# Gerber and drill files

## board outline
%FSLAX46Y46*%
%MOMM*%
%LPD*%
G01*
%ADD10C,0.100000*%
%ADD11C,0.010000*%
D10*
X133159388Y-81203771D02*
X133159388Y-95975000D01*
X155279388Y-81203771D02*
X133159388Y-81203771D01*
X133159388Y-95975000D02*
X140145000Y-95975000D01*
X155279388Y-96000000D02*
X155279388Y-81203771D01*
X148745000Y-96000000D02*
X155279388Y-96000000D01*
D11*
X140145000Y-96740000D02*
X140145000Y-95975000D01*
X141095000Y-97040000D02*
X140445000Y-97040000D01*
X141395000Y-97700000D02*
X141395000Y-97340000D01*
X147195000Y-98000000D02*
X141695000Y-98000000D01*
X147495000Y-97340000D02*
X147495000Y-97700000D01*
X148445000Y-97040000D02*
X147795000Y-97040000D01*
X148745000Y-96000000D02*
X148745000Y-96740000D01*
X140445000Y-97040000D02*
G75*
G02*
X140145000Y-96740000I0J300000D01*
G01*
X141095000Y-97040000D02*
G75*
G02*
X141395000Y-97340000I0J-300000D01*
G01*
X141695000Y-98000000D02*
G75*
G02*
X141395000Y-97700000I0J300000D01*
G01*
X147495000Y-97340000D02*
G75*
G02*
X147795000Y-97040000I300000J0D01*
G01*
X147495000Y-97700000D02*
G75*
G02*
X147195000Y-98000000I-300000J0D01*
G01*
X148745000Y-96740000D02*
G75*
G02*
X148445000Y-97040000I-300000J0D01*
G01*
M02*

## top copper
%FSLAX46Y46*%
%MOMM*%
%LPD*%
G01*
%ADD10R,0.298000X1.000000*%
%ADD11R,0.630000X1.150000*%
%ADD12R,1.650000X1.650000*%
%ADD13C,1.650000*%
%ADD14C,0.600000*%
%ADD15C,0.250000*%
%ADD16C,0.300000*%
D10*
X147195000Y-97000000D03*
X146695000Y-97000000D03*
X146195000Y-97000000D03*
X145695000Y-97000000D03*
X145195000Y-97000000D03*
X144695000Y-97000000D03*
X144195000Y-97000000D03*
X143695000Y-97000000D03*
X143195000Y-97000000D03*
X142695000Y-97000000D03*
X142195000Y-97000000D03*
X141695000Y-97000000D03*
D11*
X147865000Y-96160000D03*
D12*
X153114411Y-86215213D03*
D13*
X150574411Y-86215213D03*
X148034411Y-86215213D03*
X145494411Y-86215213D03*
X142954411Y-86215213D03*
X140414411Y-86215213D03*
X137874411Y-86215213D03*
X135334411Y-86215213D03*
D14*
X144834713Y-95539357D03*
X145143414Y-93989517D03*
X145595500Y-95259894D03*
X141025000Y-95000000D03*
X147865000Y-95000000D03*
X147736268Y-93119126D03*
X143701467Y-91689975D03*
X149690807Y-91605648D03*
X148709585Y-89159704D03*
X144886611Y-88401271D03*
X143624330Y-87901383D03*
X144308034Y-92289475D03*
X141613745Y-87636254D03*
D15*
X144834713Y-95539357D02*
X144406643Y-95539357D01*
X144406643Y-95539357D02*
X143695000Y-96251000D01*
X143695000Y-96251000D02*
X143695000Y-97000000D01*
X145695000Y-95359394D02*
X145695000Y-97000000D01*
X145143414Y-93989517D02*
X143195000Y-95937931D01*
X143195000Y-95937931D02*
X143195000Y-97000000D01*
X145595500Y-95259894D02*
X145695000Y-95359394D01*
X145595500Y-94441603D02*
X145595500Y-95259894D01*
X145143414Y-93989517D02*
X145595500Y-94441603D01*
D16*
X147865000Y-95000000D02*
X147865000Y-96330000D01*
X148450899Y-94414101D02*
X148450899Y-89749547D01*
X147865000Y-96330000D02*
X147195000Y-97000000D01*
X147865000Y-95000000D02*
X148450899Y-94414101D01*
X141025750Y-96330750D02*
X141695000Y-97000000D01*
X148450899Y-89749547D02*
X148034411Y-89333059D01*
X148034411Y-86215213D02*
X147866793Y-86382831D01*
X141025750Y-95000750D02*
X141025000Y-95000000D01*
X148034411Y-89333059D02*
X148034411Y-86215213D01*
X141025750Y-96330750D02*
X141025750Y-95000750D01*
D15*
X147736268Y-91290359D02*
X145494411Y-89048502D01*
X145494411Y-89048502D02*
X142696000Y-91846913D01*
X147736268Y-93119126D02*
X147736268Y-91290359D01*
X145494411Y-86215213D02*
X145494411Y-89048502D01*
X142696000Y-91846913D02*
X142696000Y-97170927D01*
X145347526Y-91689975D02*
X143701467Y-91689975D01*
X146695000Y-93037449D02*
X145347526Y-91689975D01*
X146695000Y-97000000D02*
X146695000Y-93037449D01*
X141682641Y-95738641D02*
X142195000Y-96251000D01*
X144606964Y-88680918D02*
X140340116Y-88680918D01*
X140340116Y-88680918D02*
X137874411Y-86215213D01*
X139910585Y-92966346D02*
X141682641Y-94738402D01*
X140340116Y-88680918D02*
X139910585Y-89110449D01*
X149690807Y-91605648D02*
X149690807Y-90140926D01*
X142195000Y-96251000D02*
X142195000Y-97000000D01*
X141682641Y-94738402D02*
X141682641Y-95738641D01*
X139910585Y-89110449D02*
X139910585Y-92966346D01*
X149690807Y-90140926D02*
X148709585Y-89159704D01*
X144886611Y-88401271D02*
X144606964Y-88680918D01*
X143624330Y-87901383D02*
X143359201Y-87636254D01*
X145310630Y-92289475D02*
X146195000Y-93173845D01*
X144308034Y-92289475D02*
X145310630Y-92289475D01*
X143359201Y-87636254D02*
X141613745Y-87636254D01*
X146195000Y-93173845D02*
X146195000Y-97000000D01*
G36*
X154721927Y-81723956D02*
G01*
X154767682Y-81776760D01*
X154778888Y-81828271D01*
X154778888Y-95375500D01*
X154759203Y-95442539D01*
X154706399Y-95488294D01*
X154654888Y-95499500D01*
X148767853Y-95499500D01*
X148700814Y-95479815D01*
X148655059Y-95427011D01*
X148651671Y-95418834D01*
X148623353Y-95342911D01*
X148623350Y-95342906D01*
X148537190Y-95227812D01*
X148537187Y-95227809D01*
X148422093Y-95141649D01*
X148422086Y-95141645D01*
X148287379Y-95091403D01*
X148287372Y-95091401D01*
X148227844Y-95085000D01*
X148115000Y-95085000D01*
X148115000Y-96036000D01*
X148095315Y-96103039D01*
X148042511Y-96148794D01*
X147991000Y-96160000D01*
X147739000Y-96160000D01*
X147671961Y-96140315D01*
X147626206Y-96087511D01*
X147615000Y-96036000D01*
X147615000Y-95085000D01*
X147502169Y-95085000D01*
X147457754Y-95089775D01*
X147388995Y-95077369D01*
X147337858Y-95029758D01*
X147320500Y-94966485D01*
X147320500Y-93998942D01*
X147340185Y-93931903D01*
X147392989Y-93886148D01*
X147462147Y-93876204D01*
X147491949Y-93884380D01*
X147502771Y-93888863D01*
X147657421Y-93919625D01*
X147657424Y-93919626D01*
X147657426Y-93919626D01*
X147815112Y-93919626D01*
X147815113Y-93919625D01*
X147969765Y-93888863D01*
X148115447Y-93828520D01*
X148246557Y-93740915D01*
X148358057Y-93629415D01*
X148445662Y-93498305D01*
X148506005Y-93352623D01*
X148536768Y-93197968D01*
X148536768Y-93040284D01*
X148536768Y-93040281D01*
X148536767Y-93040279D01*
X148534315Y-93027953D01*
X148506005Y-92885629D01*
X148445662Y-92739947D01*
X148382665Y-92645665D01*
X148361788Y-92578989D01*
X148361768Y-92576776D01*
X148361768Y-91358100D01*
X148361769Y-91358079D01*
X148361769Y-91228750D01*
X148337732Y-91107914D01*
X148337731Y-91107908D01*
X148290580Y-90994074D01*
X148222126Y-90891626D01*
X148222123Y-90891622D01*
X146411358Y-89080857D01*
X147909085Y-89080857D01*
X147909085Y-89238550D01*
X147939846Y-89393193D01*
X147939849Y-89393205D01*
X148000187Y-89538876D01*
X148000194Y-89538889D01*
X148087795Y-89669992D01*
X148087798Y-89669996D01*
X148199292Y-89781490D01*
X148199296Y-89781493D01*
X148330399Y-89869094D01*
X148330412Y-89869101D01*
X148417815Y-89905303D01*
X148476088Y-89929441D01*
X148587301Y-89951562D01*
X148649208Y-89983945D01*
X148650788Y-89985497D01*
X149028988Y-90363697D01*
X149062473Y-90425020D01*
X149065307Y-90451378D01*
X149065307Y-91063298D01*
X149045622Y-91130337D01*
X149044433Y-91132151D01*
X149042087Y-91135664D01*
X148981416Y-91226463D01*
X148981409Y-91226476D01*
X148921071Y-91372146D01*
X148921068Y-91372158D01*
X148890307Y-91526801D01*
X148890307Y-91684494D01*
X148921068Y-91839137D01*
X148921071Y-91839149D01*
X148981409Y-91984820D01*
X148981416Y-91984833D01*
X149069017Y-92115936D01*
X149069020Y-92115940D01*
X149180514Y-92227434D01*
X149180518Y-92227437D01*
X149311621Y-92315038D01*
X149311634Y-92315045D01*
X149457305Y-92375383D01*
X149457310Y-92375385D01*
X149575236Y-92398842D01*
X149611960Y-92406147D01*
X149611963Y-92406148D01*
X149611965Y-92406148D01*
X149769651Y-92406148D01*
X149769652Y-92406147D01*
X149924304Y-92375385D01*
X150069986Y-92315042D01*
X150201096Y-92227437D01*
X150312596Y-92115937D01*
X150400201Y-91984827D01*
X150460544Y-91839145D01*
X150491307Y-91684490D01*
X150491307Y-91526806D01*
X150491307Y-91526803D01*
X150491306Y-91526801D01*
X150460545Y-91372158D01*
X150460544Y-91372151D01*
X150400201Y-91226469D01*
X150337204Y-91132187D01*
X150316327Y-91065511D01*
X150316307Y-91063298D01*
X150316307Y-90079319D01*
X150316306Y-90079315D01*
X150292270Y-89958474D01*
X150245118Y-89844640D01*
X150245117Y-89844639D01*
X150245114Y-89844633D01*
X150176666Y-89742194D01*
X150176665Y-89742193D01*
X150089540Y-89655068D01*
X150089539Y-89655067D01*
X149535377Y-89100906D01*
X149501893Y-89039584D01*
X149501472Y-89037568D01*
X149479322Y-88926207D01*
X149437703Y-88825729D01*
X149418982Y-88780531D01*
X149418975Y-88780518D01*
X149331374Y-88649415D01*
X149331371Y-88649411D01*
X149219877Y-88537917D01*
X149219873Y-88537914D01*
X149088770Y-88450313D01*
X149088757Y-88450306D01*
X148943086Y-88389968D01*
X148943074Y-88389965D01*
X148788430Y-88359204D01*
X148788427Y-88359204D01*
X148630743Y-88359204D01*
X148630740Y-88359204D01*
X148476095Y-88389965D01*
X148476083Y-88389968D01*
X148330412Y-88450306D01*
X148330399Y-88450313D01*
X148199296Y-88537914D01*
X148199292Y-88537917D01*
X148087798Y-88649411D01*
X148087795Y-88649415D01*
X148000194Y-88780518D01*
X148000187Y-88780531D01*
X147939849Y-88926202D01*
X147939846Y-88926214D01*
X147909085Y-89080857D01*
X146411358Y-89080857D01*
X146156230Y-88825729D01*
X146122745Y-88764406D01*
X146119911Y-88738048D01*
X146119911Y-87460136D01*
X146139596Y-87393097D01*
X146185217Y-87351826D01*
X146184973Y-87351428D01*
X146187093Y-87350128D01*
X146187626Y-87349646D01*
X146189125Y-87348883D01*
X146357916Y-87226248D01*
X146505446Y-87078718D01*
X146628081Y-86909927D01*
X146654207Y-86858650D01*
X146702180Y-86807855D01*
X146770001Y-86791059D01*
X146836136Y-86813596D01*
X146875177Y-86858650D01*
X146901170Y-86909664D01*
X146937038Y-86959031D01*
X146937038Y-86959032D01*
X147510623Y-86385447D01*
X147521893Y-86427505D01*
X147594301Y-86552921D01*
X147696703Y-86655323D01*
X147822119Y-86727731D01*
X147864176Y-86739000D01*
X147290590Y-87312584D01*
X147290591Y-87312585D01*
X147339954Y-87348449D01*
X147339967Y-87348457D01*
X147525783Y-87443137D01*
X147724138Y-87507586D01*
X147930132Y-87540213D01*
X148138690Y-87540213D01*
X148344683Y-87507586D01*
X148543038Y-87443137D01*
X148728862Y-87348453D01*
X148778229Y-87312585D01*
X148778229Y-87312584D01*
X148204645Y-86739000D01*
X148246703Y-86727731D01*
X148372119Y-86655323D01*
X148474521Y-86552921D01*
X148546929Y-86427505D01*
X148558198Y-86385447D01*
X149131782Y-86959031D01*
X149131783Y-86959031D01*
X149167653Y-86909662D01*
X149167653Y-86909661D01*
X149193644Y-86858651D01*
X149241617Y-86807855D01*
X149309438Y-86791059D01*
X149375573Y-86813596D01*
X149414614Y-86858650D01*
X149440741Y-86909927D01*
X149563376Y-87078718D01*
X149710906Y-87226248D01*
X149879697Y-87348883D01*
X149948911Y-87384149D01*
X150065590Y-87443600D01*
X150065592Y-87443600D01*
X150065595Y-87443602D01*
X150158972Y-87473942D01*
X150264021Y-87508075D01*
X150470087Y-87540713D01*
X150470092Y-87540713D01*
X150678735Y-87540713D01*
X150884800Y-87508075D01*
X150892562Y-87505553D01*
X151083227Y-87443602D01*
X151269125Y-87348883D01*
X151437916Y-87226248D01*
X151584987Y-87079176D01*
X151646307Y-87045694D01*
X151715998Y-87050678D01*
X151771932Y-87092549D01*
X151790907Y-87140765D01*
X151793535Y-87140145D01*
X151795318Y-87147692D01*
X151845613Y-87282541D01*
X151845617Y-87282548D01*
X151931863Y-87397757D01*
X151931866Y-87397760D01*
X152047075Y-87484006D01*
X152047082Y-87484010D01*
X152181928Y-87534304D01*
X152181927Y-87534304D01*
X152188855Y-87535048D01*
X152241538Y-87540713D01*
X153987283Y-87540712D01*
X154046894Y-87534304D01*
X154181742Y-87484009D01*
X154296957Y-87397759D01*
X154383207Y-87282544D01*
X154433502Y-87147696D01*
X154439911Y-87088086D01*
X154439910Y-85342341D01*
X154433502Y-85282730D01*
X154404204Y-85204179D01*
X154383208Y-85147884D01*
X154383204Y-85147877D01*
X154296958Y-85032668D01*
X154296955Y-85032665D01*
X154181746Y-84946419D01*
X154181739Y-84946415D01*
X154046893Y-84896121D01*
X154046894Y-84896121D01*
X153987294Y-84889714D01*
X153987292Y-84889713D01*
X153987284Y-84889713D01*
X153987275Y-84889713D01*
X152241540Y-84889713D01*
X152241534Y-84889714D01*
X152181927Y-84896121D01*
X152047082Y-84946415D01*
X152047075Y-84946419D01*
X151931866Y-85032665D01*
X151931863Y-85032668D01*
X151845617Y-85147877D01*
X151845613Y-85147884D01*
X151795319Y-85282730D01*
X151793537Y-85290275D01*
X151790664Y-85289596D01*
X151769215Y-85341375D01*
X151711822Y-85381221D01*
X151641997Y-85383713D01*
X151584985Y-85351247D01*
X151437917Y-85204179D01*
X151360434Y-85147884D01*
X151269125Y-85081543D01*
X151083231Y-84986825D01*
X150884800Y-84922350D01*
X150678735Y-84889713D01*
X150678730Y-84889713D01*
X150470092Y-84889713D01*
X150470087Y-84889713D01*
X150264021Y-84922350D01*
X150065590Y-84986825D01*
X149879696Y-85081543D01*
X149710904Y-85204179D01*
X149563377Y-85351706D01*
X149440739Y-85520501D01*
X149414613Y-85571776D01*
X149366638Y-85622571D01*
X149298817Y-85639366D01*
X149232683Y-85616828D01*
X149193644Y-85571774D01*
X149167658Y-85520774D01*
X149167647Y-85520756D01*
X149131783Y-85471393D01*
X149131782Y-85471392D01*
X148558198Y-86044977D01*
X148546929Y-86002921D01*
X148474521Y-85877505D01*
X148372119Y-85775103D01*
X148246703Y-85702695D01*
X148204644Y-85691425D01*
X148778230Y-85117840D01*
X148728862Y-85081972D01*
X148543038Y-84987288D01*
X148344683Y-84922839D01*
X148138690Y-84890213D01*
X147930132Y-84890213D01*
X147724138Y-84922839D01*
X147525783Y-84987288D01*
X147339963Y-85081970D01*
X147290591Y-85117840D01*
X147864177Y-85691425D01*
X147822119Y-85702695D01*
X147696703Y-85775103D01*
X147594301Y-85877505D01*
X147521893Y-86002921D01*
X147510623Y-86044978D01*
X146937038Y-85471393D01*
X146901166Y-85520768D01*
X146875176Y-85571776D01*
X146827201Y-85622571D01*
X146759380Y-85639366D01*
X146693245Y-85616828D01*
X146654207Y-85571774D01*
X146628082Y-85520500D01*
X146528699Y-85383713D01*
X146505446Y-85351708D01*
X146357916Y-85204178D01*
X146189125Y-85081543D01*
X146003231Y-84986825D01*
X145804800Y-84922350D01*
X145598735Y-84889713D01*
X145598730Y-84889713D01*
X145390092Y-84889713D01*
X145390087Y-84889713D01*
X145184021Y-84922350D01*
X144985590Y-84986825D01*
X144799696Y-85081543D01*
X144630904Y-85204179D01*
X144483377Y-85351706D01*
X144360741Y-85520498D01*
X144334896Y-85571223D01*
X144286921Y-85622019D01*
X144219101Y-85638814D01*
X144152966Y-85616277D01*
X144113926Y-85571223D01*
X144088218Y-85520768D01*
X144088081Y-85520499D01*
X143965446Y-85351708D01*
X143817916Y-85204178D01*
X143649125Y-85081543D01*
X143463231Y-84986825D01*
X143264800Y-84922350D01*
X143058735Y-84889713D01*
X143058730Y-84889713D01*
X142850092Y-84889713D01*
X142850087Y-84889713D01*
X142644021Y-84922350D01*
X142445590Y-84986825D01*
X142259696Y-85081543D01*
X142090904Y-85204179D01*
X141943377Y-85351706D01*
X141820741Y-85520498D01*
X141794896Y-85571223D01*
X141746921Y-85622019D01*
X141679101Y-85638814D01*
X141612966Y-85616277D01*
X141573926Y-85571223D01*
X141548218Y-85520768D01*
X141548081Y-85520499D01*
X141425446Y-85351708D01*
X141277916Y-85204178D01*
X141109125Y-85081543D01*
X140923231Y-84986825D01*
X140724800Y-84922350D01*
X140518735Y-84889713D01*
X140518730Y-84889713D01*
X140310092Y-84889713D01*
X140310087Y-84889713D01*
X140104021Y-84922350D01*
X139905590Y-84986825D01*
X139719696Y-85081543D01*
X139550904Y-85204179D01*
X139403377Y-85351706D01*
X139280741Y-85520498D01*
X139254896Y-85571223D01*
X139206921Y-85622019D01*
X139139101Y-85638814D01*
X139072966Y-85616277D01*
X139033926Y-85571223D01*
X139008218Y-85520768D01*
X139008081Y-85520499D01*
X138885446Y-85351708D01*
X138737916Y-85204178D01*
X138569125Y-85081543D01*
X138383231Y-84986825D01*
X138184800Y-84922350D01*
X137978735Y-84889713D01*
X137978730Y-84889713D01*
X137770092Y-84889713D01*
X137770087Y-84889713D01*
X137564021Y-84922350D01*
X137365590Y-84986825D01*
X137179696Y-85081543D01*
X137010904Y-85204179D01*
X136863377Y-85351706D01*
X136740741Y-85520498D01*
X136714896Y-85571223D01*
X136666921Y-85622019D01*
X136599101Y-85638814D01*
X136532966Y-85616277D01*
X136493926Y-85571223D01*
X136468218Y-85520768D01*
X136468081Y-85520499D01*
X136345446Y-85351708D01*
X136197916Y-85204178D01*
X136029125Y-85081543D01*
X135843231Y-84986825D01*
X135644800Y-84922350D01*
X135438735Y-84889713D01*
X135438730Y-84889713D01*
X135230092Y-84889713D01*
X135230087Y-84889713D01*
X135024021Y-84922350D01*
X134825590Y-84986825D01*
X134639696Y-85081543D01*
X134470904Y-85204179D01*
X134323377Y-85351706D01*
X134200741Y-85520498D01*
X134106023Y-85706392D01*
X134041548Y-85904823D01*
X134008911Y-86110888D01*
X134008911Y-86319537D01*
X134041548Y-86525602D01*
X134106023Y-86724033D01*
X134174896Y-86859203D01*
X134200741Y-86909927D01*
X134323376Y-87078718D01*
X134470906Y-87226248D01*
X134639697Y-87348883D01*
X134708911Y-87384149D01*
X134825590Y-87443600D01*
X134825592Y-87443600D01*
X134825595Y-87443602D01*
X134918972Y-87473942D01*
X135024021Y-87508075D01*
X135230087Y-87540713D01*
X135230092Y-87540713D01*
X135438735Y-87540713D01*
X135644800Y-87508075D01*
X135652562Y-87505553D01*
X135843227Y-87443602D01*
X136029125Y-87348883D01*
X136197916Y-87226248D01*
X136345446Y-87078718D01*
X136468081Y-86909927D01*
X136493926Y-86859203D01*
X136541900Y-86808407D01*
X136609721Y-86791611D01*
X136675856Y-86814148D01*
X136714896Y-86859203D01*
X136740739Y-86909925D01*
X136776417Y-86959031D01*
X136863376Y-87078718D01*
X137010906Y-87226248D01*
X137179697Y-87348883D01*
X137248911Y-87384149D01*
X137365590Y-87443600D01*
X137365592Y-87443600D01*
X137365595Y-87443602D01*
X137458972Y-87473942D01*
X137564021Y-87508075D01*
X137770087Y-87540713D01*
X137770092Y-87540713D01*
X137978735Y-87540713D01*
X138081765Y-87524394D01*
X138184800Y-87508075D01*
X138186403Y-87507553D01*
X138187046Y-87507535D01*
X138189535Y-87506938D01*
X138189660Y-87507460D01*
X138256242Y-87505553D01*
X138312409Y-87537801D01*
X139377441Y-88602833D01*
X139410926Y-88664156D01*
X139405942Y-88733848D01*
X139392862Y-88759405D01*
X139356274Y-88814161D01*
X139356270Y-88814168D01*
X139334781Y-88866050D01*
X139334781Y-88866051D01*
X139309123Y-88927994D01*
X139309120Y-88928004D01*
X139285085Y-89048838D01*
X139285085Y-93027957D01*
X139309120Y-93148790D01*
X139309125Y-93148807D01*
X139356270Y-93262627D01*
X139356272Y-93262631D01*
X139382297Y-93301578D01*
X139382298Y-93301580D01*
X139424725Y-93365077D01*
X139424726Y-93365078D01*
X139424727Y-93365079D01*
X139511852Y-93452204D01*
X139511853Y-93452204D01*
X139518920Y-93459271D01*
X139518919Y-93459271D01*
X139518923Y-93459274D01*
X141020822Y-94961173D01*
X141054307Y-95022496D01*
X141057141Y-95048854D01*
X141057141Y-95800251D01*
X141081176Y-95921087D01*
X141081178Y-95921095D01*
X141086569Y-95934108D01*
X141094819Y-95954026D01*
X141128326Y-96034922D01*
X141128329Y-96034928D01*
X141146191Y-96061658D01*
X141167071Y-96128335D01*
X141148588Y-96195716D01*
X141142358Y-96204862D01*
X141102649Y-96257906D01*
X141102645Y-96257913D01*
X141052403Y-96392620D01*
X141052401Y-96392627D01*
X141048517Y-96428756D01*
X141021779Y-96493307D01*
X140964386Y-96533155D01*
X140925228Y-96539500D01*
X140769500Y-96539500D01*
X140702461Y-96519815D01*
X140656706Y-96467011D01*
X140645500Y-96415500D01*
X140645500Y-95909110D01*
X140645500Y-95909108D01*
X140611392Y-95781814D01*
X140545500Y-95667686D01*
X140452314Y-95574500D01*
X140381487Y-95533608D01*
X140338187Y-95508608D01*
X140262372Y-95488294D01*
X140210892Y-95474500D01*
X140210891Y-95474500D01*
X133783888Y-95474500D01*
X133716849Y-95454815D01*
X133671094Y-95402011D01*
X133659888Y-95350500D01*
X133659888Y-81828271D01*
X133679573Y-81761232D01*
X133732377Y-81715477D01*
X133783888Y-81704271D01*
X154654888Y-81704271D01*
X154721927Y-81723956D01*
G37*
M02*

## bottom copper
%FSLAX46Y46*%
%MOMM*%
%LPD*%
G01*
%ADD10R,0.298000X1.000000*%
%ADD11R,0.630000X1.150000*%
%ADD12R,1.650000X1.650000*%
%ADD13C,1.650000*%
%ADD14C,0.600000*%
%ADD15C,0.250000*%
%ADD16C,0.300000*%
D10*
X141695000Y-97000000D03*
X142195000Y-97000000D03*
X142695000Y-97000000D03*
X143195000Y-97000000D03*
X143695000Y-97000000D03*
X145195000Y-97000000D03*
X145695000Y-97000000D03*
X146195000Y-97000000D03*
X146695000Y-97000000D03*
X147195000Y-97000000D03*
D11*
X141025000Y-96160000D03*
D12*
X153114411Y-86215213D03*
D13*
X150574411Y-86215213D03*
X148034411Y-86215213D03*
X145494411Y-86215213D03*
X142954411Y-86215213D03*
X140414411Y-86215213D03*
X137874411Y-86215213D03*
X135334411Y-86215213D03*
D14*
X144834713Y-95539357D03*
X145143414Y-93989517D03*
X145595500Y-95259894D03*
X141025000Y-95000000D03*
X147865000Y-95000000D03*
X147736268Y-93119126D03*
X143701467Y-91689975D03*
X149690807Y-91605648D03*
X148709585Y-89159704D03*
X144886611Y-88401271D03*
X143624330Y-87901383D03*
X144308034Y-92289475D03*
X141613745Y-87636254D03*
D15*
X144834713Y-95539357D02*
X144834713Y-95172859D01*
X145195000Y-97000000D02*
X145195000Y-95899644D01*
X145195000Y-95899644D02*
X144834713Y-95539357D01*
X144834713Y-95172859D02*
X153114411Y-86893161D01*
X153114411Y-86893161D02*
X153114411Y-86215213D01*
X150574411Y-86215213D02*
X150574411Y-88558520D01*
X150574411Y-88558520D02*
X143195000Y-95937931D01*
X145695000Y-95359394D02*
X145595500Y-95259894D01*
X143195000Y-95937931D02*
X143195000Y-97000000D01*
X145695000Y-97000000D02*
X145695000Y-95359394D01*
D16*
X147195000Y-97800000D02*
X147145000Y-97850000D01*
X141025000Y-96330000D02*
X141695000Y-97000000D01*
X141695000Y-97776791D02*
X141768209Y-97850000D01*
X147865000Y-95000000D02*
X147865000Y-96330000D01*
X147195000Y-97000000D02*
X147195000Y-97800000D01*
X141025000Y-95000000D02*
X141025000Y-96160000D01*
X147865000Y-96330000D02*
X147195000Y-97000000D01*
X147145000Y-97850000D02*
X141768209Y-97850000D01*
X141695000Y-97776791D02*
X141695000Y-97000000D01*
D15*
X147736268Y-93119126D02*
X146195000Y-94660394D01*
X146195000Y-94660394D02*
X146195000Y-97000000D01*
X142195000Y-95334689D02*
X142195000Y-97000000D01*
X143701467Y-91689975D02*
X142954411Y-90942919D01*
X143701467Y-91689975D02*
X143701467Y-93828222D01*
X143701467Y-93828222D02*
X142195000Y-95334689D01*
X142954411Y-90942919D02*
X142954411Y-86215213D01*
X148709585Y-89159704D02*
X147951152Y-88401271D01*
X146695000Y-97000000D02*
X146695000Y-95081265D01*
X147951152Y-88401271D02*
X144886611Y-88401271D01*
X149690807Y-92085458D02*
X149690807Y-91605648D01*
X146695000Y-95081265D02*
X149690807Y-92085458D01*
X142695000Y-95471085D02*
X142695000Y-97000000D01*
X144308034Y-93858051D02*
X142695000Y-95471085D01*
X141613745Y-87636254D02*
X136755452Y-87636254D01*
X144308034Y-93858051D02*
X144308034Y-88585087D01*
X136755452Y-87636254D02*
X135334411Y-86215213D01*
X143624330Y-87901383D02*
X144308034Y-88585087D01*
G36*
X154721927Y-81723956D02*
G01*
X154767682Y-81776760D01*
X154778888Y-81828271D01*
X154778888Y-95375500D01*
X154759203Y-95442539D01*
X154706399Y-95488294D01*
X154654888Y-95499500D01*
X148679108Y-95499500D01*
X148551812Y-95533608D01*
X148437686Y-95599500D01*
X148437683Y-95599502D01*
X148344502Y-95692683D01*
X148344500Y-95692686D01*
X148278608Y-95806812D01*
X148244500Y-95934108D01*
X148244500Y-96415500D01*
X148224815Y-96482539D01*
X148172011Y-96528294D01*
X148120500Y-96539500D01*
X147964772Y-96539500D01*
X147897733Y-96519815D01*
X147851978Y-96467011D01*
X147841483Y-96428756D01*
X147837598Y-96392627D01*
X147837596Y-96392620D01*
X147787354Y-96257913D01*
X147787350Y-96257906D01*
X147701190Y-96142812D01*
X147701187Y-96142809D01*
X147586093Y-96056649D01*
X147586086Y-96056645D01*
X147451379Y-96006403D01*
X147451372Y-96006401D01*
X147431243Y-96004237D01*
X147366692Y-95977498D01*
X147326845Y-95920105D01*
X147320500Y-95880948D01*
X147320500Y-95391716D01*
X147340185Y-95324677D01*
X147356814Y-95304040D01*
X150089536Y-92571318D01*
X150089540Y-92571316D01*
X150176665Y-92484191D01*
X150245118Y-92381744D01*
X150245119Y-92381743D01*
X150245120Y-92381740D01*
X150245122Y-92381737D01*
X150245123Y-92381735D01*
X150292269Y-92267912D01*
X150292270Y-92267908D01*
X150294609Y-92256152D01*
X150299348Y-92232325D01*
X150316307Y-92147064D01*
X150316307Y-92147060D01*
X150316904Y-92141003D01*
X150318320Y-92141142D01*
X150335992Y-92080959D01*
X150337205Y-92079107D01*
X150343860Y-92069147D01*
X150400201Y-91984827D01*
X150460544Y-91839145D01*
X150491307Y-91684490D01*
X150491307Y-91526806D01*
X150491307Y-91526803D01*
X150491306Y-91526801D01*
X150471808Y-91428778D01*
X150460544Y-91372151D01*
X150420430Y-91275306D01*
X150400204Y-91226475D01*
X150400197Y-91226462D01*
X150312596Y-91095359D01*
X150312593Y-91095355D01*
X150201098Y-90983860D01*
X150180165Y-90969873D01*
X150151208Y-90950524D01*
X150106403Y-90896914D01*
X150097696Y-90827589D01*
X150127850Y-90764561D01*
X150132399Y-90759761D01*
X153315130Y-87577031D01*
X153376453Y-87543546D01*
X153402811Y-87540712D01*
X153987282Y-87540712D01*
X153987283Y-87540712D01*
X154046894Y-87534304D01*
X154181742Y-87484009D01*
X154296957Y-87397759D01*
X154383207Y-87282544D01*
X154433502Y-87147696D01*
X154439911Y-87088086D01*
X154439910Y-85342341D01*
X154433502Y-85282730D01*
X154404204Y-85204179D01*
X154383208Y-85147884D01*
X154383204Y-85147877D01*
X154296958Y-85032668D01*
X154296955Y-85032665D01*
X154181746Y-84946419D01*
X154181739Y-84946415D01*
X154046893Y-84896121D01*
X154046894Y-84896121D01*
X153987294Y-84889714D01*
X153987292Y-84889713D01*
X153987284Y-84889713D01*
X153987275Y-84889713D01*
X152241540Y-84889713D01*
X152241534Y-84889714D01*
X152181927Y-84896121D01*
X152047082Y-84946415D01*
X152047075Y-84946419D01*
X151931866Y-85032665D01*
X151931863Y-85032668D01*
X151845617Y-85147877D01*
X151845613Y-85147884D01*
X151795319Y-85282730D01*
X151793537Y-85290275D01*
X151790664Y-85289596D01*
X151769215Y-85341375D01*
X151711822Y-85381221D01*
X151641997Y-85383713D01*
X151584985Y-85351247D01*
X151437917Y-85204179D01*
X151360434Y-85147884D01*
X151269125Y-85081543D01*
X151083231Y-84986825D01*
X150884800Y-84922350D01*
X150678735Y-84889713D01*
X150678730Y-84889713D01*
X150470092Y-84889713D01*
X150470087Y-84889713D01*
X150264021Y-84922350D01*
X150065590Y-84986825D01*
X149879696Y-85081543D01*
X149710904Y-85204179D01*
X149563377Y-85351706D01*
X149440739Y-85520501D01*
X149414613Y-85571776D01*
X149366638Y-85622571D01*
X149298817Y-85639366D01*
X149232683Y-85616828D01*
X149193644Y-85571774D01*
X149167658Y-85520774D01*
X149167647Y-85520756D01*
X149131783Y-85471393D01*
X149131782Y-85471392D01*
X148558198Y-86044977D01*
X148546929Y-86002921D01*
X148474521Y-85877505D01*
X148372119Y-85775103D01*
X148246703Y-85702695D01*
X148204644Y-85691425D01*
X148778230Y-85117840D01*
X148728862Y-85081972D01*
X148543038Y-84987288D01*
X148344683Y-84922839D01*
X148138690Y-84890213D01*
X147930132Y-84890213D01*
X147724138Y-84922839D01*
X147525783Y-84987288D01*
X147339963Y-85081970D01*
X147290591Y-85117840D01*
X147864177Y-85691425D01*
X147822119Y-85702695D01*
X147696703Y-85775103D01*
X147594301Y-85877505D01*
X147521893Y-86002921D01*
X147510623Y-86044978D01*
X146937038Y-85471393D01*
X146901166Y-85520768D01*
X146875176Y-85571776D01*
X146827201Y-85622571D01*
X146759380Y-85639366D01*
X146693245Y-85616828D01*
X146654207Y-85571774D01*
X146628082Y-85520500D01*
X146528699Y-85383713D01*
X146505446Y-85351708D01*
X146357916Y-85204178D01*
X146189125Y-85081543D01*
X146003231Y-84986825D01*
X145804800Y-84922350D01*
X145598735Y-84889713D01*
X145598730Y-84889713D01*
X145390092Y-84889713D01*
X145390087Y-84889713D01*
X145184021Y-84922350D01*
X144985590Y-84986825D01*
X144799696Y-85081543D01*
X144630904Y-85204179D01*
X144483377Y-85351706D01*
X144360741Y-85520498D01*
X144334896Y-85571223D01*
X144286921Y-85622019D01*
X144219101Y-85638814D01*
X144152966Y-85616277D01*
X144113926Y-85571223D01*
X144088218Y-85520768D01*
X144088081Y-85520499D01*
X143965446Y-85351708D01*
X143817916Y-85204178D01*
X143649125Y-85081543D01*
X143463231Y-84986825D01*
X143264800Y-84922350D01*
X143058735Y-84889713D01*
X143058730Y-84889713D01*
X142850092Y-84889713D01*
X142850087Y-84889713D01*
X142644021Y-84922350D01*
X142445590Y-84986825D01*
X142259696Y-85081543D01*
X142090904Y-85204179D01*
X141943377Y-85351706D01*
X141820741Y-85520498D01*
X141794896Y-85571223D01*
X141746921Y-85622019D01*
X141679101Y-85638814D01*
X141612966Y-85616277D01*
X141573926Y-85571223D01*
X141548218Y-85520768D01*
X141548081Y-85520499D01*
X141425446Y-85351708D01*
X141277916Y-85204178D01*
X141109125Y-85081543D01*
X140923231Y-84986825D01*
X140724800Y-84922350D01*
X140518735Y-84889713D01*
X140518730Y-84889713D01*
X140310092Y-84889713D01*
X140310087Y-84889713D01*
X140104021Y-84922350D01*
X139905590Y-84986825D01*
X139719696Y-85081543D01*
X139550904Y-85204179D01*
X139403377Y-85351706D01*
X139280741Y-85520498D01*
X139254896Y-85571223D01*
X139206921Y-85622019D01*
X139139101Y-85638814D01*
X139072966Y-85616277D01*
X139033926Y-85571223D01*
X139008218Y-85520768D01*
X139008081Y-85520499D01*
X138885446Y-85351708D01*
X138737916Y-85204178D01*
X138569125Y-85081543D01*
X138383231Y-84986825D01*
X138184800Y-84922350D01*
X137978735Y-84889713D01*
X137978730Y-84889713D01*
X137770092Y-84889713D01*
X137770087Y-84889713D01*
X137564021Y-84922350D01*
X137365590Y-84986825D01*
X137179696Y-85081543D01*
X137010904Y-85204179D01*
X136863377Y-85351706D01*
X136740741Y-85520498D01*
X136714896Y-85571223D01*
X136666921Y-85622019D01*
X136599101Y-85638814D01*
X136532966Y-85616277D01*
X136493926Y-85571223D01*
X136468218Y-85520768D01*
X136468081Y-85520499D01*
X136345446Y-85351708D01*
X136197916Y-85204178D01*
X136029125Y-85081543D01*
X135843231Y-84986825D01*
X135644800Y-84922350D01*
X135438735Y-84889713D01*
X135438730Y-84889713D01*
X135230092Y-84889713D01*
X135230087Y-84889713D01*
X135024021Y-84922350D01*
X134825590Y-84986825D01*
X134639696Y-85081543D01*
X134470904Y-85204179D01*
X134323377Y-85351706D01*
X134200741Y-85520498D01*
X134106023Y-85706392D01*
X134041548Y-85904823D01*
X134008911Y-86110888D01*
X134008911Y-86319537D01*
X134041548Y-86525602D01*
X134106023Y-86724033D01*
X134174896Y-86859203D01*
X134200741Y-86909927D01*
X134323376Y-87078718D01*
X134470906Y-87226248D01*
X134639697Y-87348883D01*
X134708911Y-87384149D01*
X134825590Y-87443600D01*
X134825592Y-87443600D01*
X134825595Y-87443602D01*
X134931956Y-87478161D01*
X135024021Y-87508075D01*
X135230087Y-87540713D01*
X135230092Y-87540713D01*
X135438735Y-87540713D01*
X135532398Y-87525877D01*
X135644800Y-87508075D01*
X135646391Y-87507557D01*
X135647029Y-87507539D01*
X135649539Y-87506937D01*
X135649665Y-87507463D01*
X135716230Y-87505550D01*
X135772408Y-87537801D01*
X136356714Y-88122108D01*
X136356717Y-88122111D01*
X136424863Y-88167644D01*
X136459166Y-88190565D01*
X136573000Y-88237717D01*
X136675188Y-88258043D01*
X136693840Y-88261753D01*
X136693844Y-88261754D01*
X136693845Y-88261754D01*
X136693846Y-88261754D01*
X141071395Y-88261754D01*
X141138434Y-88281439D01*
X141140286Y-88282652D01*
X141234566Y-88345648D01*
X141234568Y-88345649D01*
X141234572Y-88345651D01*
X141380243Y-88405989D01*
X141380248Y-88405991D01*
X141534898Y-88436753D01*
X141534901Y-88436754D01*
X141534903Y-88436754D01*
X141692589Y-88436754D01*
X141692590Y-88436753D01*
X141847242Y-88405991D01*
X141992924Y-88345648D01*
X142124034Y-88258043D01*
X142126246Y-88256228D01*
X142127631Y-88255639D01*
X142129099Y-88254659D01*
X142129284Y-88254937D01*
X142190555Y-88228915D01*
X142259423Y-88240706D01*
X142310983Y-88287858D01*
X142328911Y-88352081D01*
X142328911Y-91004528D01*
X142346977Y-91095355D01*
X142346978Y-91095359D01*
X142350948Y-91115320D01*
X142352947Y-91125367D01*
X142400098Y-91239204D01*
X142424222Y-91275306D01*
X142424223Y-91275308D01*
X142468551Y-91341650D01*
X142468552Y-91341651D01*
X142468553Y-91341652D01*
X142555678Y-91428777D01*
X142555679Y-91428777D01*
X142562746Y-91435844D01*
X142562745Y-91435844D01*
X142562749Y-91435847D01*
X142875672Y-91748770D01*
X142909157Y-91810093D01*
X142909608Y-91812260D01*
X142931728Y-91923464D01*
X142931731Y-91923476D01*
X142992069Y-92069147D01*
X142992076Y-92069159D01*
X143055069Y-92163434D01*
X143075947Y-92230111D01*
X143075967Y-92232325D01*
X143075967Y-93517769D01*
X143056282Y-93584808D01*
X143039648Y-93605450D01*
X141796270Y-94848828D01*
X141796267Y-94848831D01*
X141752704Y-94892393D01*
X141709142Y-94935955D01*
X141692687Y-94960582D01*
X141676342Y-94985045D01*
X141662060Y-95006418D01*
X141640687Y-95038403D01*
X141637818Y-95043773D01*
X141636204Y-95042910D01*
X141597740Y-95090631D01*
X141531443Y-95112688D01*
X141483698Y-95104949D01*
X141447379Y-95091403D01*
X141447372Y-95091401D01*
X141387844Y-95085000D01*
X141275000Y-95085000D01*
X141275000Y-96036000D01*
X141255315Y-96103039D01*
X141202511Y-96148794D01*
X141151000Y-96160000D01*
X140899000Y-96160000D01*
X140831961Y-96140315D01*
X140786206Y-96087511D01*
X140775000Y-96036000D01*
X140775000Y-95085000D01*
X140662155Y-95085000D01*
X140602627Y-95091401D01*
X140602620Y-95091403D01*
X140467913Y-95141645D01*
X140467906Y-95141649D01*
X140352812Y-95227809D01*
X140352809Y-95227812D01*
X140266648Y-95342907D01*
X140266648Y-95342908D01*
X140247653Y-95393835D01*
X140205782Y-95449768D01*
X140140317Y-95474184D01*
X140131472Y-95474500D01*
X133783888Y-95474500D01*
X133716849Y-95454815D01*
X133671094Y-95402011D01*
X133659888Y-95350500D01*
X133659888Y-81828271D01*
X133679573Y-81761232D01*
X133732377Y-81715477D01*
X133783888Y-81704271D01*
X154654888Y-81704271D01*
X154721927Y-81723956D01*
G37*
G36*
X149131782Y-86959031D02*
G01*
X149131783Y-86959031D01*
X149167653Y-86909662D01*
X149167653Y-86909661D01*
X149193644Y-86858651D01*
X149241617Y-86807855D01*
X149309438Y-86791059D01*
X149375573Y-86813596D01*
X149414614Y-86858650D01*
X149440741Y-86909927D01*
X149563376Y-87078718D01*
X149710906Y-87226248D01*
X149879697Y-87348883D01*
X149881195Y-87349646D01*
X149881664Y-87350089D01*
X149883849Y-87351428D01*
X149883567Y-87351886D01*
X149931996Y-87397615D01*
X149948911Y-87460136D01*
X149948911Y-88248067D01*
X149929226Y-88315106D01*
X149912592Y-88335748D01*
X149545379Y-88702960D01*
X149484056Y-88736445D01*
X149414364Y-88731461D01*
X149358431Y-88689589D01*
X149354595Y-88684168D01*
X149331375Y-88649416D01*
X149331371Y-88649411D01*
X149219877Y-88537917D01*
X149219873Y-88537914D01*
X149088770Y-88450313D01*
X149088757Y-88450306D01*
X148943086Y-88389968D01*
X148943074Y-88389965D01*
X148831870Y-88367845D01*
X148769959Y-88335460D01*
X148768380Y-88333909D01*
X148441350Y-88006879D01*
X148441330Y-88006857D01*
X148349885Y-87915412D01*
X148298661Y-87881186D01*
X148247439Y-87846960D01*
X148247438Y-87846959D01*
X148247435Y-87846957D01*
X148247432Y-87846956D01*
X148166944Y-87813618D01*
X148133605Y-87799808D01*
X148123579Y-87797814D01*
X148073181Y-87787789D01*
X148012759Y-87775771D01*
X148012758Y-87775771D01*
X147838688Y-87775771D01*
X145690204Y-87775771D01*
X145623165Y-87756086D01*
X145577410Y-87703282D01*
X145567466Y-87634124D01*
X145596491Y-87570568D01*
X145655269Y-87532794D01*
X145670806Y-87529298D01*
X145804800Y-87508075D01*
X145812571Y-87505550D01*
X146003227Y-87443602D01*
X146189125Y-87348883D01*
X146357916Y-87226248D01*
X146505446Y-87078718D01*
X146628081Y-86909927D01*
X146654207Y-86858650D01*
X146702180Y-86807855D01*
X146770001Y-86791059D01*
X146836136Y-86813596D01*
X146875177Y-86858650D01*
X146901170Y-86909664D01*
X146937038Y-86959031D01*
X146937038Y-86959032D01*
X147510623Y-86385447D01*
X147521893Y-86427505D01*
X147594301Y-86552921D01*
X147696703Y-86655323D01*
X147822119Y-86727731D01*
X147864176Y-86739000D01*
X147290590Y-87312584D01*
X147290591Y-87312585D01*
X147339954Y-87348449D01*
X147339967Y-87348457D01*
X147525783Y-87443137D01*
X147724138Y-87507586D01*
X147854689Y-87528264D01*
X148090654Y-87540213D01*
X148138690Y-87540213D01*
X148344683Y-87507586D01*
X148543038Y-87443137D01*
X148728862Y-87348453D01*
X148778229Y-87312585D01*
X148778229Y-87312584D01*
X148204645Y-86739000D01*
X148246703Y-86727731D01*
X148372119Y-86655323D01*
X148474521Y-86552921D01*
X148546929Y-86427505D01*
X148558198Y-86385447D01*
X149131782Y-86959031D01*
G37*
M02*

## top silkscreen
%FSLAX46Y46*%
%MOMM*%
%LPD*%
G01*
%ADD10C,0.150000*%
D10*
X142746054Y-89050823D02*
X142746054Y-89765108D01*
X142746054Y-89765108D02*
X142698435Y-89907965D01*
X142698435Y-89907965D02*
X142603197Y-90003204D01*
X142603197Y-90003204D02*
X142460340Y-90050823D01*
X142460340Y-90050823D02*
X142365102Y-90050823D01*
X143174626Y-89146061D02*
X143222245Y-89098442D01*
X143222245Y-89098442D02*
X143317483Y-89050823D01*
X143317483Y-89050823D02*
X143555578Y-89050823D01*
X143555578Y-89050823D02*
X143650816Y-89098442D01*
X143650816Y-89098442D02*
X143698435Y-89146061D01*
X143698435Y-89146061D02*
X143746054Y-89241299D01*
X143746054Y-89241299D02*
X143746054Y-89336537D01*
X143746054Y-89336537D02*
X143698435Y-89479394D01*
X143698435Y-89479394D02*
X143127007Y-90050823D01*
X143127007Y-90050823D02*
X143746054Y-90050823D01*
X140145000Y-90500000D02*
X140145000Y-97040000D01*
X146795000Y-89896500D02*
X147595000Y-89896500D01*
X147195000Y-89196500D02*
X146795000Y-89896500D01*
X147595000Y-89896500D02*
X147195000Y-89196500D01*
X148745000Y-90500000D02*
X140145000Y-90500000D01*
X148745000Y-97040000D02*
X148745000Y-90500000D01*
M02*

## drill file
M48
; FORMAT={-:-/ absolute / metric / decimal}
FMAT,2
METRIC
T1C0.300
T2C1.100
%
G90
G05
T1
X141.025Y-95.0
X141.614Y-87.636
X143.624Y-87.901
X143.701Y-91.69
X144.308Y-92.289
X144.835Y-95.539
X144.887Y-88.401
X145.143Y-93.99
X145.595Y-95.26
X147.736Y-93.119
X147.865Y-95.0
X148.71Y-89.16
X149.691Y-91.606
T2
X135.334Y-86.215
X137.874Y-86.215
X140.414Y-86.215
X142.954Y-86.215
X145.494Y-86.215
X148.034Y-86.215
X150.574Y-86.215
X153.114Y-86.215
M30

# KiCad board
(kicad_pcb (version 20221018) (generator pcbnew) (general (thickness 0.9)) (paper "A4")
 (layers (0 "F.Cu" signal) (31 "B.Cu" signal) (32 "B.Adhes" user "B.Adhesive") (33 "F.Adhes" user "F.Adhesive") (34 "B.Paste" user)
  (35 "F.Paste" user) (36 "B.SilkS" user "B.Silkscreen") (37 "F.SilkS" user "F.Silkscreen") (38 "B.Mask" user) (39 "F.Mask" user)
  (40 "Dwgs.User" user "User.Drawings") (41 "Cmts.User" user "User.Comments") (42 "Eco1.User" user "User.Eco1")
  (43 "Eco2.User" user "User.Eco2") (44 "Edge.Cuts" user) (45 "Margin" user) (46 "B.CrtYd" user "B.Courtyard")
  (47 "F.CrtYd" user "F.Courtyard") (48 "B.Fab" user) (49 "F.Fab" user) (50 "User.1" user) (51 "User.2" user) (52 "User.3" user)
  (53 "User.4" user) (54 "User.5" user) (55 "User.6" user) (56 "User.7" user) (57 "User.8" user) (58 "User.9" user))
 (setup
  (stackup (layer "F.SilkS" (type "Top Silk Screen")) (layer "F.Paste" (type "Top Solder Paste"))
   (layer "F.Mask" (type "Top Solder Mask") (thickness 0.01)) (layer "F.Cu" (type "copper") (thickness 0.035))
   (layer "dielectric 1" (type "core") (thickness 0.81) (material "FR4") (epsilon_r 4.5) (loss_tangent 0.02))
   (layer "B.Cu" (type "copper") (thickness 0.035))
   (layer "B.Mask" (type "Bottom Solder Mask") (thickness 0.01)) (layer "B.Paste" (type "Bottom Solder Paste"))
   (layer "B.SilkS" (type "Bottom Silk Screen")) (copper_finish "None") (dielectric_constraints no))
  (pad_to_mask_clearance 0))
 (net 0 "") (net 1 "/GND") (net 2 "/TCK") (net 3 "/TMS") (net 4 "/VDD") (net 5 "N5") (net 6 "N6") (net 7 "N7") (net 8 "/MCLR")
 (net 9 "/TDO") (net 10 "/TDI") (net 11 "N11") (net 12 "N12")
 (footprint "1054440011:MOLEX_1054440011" (layer "F.Cu") (at 144.445 98)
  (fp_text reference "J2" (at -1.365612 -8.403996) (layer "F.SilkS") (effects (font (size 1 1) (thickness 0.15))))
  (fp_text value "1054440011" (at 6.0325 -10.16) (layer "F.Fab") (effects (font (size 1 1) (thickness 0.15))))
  (fp_line (start -4.3 -7.5) (end -4.3 -0.96) (stroke (width 0.15) (type solid)) (layer "F.SilkS"))
  (fp_line (start 2.35 -8.1035) (end 3.15 -8.1035) (stroke (width 0.15) (type solid)) (layer "F.SilkS"))
  (fp_line (start 2.75 -8.8035) (end 2.35 -8.1035) (stroke (width 0.15) (type solid)) (layer "F.SilkS"))
  (fp_line (start 3.15 -8.1035) (end 2.75 -8.8035) (stroke (width 0.15) (type solid)) (layer "F.SilkS"))
  (fp_line (start 4.3 -7.5) (end -4.3 -7.5) (stroke (width 0.15) (type solid)) (layer "F.SilkS"))
  (fp_line (start 4.3 -0.96) (end 4.3 -7.5) (stroke (width 0.15) (type solid)) (layer "F.SilkS"))
  (fp_line (start -4.3 -1.26) (end -4.3 -2.025) (stroke (width 0.01) (type solid)) (layer "Edge.Cuts"))
  (fp_line (start -3.35 -0.96) (end -4 -0.96) (stroke (width 0.01) (type solid)) (layer "Edge.Cuts"))
  (fp_line (start -3.05 -0.3) (end -3.05 -0.66) (stroke (width 0.01) (type solid)) (layer "Edge.Cuts"))
  (fp_line (start 2.75 0) (end -2.75 0) (stroke (width 0.01) (type solid)) (layer "Edge.Cuts"))
  (fp_line (start 3.05 -0.66) (end 3.05 -0.3) (stroke (width 0.01) (type solid)) (layer "Edge.Cuts"))
  (fp_line (start 4 -0.96) (end 3.35 -0.96) (stroke (width 0.01) (type solid)) (layer "Edge.Cuts"))
  (fp_line (start 4.3 -2) (end 4.3 -1.26) (stroke (width 0.01) (type solid)) (layer "Edge.Cuts"))
  (fp_arc (start -4 -0.96) (mid -4.212132 -1.047868) (end -4.3 -1.26) (stroke (width 0.01) (type solid)) (layer "Edge.Cuts"))
  (fp_arc (start -3.35 -0.96) (mid -3.137868 -0.872132) (end -3.05 -0.66) (stroke (width 0.01) (type solid)) (layer "Edge.Cuts"))
  (fp_arc (start -2.75 0) (mid -2.962132 -0.087868) (end -3.05 -0.3) (stroke (width 0.01) (type solid)) (layer "Edge.Cuts"))
  (fp_arc (start 3.05 -0.66) (mid 3.137868 -0.872132) (end 3.35 -0.96) (stroke (width 0.01) (type solid)) (layer "Edge.Cuts"))
  (fp_arc (start 3.05 -0.3) (mid 2.962132 -0.087868) (end 2.75 0) (stroke (width 0.01) (type solid)) (layer "Edge.Cuts"))
  (fp_arc (start 4.3 -1.26) (mid 4.212132 -1.047868) (end 4 -0.96) (stroke (width 0.01) (type solid)) (layer "Edge.Cuts"))
  (pad "A1" smd rect (at 2.75 -1) (size 0.298 1) (layers "F.Cu" "F.Paste") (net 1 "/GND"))
  (pad "A2" smd rect (at 2.25 -1) (size 0.298 1) (layers "F.Cu" "F.Paste") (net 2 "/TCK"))
  (pad "A3" smd rect (at 1.75 -1) (size 0.298 1) (layers "F.Cu" "F.Paste") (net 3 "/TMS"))
  (pad "A4" smd rect (at 1.25 -1) (size 0.298 1) (layers "F.Cu" "F.Paste") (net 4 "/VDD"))
  (pad "A5" smd rect (at 0.75 -1) (size 0.298 1) (layers "F.Cu" "F.Paste") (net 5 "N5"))
  (pad "A6" smd rect (at 0.25 -1) (size 0.298 1) (layers "F.Cu" "F.Paste") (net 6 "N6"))
  (pad "A7" smd rect (at -0.25 -1) (size 0.298 1) (layers "F.Cu" "F.Paste") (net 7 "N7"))
  (pad "A8" smd rect (at -0.75 -1) (size 0.298 1) (layers "F.Cu" "F.Paste") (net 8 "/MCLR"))
  (pad "A9" smd rect (at -1.25 -1) (size 0.298 1) (layers "F.Cu" "F.Paste") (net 4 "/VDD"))
  (pad "A10" smd rect (at -1.75 -1) (size 0.298 1) (layers "F.Cu" "F.Paste") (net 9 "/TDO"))
  (pad "A11" smd rect (at -2.25 -1) (size 0.298 1) (layers "F.Cu" "F.Paste") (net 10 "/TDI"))
  (pad "A12" smd rect (at -2.75 -1) (size 0.298 1) (layers "F.Cu" "F.Paste") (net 1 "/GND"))
  (pad "B1" smd rect (at -2.75 -1) (size 0.298 1) (layers "B.Cu" "B.Paste") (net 1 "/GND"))
  (pad "B2" smd rect (at -2.25 -1) (size 0.298 1) (layers "B.Cu" "B.Paste") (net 2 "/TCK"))
  (pad "B3" smd rect (at -1.75 -1) (size 0.298 1) (layers "B.Cu" "B.Paste") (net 3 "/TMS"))
  (pad "B4" smd rect (at -1.25 -1) (size 0.298 1) (layers "B.Cu" "B.Paste") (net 4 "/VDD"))
  (pad "B5" smd rect (at -0.75 -1) (size 0.298 1) (layers "B.Cu" "B.Paste") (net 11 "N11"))
  (pad "B8" smd rect (at 0.75 -1) (size 0.298 1) (layers "B.Cu" "B.Paste") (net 8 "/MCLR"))
  (pad "B9" smd rect (at 1.25 -1) (size 0.298 1) (layers "B.Cu" "B.Paste") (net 4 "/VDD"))
  (pad "B10" smd rect (at 1.75 -1) (size 0.298 1) (layers "B.Cu" "B.Paste") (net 9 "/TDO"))
  (pad "B11" smd rect (at 2.25 -1) (size 0.298 1) (layers "B.Cu" "B.Paste") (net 10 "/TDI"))
  (pad "B12" smd rect (at 2.75 -1) (size 0.298 1) (layers "B.Cu" "B.Paste") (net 1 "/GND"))
  (pad "SH1" smd rect (at 3.42 -1.84) (size 0.63 1.15) (layers "F.Cu" "F.Paste") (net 1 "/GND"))
  (pad "SH2" smd rect (at -3.42 -1.84) (size 0.63 1.15) (layers "B.Cu" "B.Paste") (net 1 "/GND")))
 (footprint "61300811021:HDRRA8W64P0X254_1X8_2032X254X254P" (layer "B.Cu") (at 153.114411 86.215213 180)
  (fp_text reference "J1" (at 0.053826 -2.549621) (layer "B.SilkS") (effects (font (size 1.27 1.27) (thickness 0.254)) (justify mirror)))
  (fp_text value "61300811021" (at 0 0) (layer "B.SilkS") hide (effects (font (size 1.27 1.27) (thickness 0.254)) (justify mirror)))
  (pad "1" thru_hole rect (at 0 0 180) (size 1.65 1.65) (drill 1.1) (layers "*.Cu" "*.Mask") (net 8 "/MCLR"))
  (pad "2" thru_hole circle (at 2.54 0 180) (size 1.65 1.65) (drill 1.1) (layers "*.Cu" "*.Mask") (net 4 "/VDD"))
  (pad "3" thru_hole circle (at 5.08 0 180) (size 1.65 1.65) (drill 1.1) (layers "*.Cu" "*.Mask") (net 1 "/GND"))
  (pad "4" thru_hole circle (at 7.62 0 180) (size 1.65 1.65) (drill 1.1) (layers "*.Cu" "*.Mask") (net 9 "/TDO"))
  (pad "5" thru_hole circle (at 10.16 0 180) (size 1.65 1.65) (drill 1.1) (layers "*.Cu" "*.Mask") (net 2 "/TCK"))
  (pad "6" thru_hole circle (at 12.7 0 180) (size 1.65 1.65) (drill 1.1) (layers "*.Cu" "*.Mask") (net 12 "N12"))
  (pad "7" thru_hole circle (at 15.24 0 180) (size 1.65 1.65) (drill 1.1) (layers "*.Cu" "*.Mask") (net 10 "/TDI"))
  (pad "8" thru_hole circle (at 17.78 0 180) (size 1.65 1.65) (drill 1.1) (layers "*.Cu" "*.Mask") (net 3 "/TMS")))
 (gr_line (start 133.159388 81.203771) (end 133.159388 95.975) (stroke (width 0.1) (type default)) (layer "Edge.Cuts"))
 (gr_line (start 155.279388 81.203771) (end 133.159388 81.203771) (stroke (width 0.1) (type default)) (layer "Edge.Cuts"))
 (gr_line (start 133.159388 95.975) (end 140.145 95.975) (stroke (width 0.1) (type default)) (layer "Edge.Cuts"))
 (gr_line (start 155.279388 96) (end 155.279388 81.203771) (stroke (width 0.1) (type default)) (layer "Edge.Cuts"))
 (gr_line (start 148.745 96) (end 155.279388 96) (stroke (width 0.1) (type default)) (layer "Edge.Cuts"))
 (segment (start 144.834713 95.539357) (end 144.406643 95.539357) (width 0.25) (layer "F.Cu") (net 8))
 (segment (start 144.406643 95.539357) (end 143.695 96.251) (width 0.25) (layer "F.Cu") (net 8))
 (segment (start 143.695 96.251) (end 143.695 97) (width 0.25) (layer "F.Cu") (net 8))
 (via (at 144.834713 95.539357) (size 0.6) (drill 0.3) (layers "F.Cu" "B.Cu") (free) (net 8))
 (segment (start 144.834713 95.539357) (end 144.834713 95.172859) (width 0.25) (layer "B.Cu") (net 8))
 (segment (start 145.195 97) (end 145.195 95.899644) (width 0.25) (layer "B.Cu") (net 8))
 (segment (start 145.195 95.899644) (end 144.834713 95.539357) (width 0.25) (layer "B.Cu") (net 8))
 (segment (start 144.834713 95.172859) (end 153.114411 86.893161) (width 0.25) (layer "B.Cu") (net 8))
 (segment (start 153.114411 86.893161) (end 153.114411 86.215213) (width 0.25) (layer "B.Cu") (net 8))
 (segment (start 145.695 95.359394) (end 145.695 97) (width 0.25) (layer "F.Cu") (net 4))
 (segment (start 145.143414 93.989517) (end 143.195 95.937931) (width 0.25) (layer "F.Cu") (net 4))
 (segment (start 143.195 95.937931) (end 143.195 97) (width 0.25) (layer "F.Cu") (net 4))
 (segment (start 145.5955 95.259894) (end 145.695 95.359394) (width 0.25) (layer "F.Cu") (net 4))
 (segment (start 145.5955 94.441603) (end 145.5955 95.259894) (width 0.25) (layer "F.Cu") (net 4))
 (segment (start 145.143414 93.989517) (end 145.5955 94.441603) (width 0.25) (layer "F.Cu") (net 4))
 (via (at 145.143414 93.989517) (size 0.6) (drill 0.3) (layers "F.Cu" "B.Cu") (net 4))
 (via (at 145.5955 95.259894) (size 0.6) (drill 0.3) (layers "F.Cu" "B.Cu") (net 4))
 (segment (start 150.574411 86.215213) (end 150.574411 88.55852) (width 0.25) (layer "B.Cu") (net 4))
 (segment (start 150.574411 88.55852) (end 143.195 95.937931) (width 0.25) (layer "B.Cu") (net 4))
 (segment (start 145.695 95.359394) (end 145.5955 95.259894) (width 0.25) (layer "B.Cu") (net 4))
 (segment (start 143.195 95.937931) (end 143.195 97) (width 0.25) (layer "B.Cu") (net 4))
 (segment (start 145.695 97) (end 145.695 95.359394) (width 0.25) (layer "B.Cu") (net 4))
 (segment (start 147.865 95) (end 147.865 96.33) (width 0.3) (layer "F.Cu") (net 1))
 (segment (start 148.450899 94.414101) (end 148.450899 89.749547) (width 0.3) (layer "F.Cu") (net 1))
 (segment (start 147.865 96.33) (end 147.195 97) (width 0.3) (layer "F.Cu") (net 1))
 (segment (start 147.865 95) (end 148.450899 94.414101) (width 0.3) (layer "F.Cu") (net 1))
 (segment (start 141.02575 96.33075) (end 141.695 97) (width 0.3) (layer "F.Cu") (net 1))
 (segment (start 148.450899 89.749547) (end 148.034411 89.333059) (width 0.3) (layer "F.Cu") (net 1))
 (segment (start 148.034411 86.215213) (end 147.866793 86.382831) (width 0.3) (layer "F.Cu") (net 1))
 (segment (start 141.02575 95.00075) (end 141.025 95) (width 0.3) (layer "F.Cu") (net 1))
 (segment (start 148.034411 89.333059) (end 148.034411 86.215213) (width 0.3) (layer "F.Cu") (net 1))
 (segment (start 141.02575 96.33075) (end 141.02575 95.00075) (width 0.3) (layer "F.Cu") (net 1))
 (via (at 141.025 95) (size 0.6) (drill 0.3) (layers "F.Cu" "B.Cu") (free) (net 1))
 (via (at 147.865 95) (size 0.6) (drill 0.3) (layers "F.Cu" "B.Cu") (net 1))
 (segment (start 147.195 97.8) (end 147.145 97.85) (width 0.3) (layer "B.Cu") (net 1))
 (segment (start 141.025 96.33) (end 141.695 97) (width 0.3) (layer "B.Cu") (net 1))
 (segment (start 141.695 97.776791) (end 141.768209 97.85) (width 0.3) (layer "B.Cu") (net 1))
 (segment (start 147.865 95) (end 147.865 96.33) (width 0.3) (layer "B.Cu") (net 1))
 (segment (start 147.195 97) (end 147.195 97.8) (width 0.3) (layer "B.Cu") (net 1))
 (segment (start 141.025 95) (end 141.025 96.16) (width 0.3) (layer "B.Cu") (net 1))
 (segment (start 147.865 96.33) (end 147.195 97) (width 0.3) (layer "B.Cu") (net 1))
 (segment (start 147.145 97.85) (end 141.768209 97.85) (width 0.3) (layer "B.Cu") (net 1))
 (segment (start 141.695 97.776791) (end 141.695 97) (width 0.3) (layer "B.Cu") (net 1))
 (segment (start 147.736268 91.290359) (end 145.494411 89.048502) (width 0.25) (layer "F.Cu") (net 9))
 (segment (start 145.494411 89.048502) (end 142.696 91.846913) (width 0.25) (layer "F.Cu") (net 9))
 (segment (start 147.736268 93.119126) (end 147.736268 91.290359) (width 0.25) (layer "F.Cu") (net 9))
 (segment (start 145.494411 86.215213) (end 145.494411 89.048502) (width 0.25) (layer "F.Cu") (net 9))
 (segment (start 142.696 91.846913) (end 142.696 97.170927) (width 0.25) (layer "F.Cu") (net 9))
 (via (at 147.736268 93.119126) (size 0.6) (drill 0.3) (layers "F.Cu" "B.Cu") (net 9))
 (segment (start 147.736268 93.119126) (end 146.195 94.660394) (width 0.25) (layer "B.Cu") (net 9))
 (segment (start 146.195 94.660394) (end 146.195 97) (width 0.25) (layer "B.Cu") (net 9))
 (segment (start 145.347526 91.689975) (end 143.701467 91.689975) (width 0.25) (layer "F.Cu") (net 2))
 (segment (start 146.695 93.037449) (end 145.347526 91.689975) (width 0.25) (layer "F.Cu") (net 2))
 (segment (start 146.695 97) (end 146.695 93.037449) (width 0.25) (layer "F.Cu") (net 2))
 (via (at 143.701467 91.689975) (size 0.6) (drill 0.3) (layers "F.Cu" "B.Cu") (free) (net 2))
 (segment (start 142.195 95.334689) (end 142.195 97) (width 0.25) (layer "B.Cu") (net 2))
 (segment (start 143.701467 91.689975) (end 142.954411 90.942919) (width 0.25) (layer "B.Cu") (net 2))
 (segment (start 143.701467 91.689975) (end 143.701467 93.828222) (width 0.25) (layer "B.Cu") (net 2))
 (segment (start 143.701467 93.828222) (end 142.195 95.334689) (width 0.25) (layer "B.Cu") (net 2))
 (segment (start 142.954411 90.942919) (end 142.954411 86.215213) (width 0.25) (layer "B.Cu") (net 2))
 (segment (start 141.682641 95.738641) (end 142.195 96.251) (width 0.25) (layer "F.Cu") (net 10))
 (segment (start 144.606964 88.680918) (end 140.340116 88.680918) (width 0.25) (layer "F.Cu") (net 10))
 (segment (start 140.340116 88.680918) (end 137.874411 86.215213) (width 0.25) (layer "F.Cu") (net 10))
 (segment (start 139.910585 92.966346) (end 141.682641 94.738402) (width 0.25) (layer "F.Cu") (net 10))
 (segment (start 140.340116 88.680918) (end 139.910585 89.110449) (width 0.25) (layer "F.Cu") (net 10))
 (segment (start 149.690807 91.605648) (end 149.690807 90.140926) (width 0.25) (layer "F.Cu") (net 10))
 (segment (start 142.195 96.251) (end 142.195 97) (width 0.25) (layer "F.Cu") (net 10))
 (segment (start 141.682641 94.738402) (end 141.682641 95.738641) (width 0.25) (layer "F.Cu") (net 10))
 (segment (start 139.910585 89.110449) (end 139.910585 92.966346) (width 0.25) (layer "F.Cu") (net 10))
 (segment (start 149.690807 90.140926) (end 148.709585 89.159704) (width 0.25) (layer "F.Cu") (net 10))
 (segment (start 144.886611 88.401271) (end 144.606964 88.680918) (width 0.25) (layer "F.Cu") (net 10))
 (via (at 149.690807 91.605648) (size 0.6) (drill 0.3) (layers "F.Cu" "B.Cu") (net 10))
 (via (at 148.709585 89.159704) (size 0.6) (drill 0.3) (layers "F.Cu" "B.Cu") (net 10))
 (via (at 144.886611 88.401271) (size 0.6) (drill 0.3) (layers "F.Cu" "B.Cu") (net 10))
 (segment (start 148.709585 89.159704) (end 147.951152 88.401271) (width 0.25) (layer "B.Cu") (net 10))
 (segment (start 146.695 97) (end 146.695 95.081265) (width 0.25) (layer "B.Cu") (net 10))
 (segment (start 147.951152 88.401271) (end 144.886611 88.401271) (width 0.25) (layer "B.Cu") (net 10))
 (segment (start 149.690807 92.085458) (end 149.690807 91.605648) (width 0.25) (layer "B.Cu") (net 10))
 (segment (start 146.695 95.081265) (end 149.690807 92.085458) (width 0.25) (layer "B.Cu") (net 10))
 (segment (start 143.62433 87.901383) (end 143.359201 87.636254) (width 0.25) (layer "F.Cu") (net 3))
 (segment (start 145.31063 92.289475) (end 146.195 93.173845) (width 0.25) (layer "F.Cu") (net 3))
 (segment (start 144.308034 92.289475) (end 145.31063 92.289475) (width 0.25) (layer "F.Cu") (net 3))
 (segment (start 143.359201 87.636254) (end 141.613745 87.636254) (width 0.25) (layer "F.Cu") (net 3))
 (segment (start 146.195 93.173845) (end 146.195 97) (width 0.25) (layer "F.Cu") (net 3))
 (via (at 143.62433 87.901383) (size 0.6) (drill 0.3) (layers "F.Cu" "B.Cu") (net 3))
 (via (at 144.308034 92.289475) (size 0.6) (drill 0.3) (layers "F.Cu" "B.Cu") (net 3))
 (via (at 141.613745 87.636254) (size 0.6) (drill 0.3) (layers "F.Cu" "B.Cu") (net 3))
 (segment (start 142.695 95.471085) (end 142.695 97) (width 0.25) (layer "B.Cu") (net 3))
 (segment (start 144.308034 93.858051) (end 142.695 95.471085) (width 0.25) (layer "B.Cu") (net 3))
 (segment (start 141.613745 87.636254) (end 136.755452 87.636254) (width 0.25) (layer "B.Cu") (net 3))
 (segment (start 144.308034 93.858051) (end 144.308034 88.585087) (width 0.25) (layer "B.Cu") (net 3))
 (segment (start 136.755452 87.636254) (end 135.334411 86.215213) (width 0.25) (layer "B.Cu") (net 3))
 (segment (start 143.62433 87.901383) (end 144.308034 88.585087) (width 0.25) (layer "B.Cu") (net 3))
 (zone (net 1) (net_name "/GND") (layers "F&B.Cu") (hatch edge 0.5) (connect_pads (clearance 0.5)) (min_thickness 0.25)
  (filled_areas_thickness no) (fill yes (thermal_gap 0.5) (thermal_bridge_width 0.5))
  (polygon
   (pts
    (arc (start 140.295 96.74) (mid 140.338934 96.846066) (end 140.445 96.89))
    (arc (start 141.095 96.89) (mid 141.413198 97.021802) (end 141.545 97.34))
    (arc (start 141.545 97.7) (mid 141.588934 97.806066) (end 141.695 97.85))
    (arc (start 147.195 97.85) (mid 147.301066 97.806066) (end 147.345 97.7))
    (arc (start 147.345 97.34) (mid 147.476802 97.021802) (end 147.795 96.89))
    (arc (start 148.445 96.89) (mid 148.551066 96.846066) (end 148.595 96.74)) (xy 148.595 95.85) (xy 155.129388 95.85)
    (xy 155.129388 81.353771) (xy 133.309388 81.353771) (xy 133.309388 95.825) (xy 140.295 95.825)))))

